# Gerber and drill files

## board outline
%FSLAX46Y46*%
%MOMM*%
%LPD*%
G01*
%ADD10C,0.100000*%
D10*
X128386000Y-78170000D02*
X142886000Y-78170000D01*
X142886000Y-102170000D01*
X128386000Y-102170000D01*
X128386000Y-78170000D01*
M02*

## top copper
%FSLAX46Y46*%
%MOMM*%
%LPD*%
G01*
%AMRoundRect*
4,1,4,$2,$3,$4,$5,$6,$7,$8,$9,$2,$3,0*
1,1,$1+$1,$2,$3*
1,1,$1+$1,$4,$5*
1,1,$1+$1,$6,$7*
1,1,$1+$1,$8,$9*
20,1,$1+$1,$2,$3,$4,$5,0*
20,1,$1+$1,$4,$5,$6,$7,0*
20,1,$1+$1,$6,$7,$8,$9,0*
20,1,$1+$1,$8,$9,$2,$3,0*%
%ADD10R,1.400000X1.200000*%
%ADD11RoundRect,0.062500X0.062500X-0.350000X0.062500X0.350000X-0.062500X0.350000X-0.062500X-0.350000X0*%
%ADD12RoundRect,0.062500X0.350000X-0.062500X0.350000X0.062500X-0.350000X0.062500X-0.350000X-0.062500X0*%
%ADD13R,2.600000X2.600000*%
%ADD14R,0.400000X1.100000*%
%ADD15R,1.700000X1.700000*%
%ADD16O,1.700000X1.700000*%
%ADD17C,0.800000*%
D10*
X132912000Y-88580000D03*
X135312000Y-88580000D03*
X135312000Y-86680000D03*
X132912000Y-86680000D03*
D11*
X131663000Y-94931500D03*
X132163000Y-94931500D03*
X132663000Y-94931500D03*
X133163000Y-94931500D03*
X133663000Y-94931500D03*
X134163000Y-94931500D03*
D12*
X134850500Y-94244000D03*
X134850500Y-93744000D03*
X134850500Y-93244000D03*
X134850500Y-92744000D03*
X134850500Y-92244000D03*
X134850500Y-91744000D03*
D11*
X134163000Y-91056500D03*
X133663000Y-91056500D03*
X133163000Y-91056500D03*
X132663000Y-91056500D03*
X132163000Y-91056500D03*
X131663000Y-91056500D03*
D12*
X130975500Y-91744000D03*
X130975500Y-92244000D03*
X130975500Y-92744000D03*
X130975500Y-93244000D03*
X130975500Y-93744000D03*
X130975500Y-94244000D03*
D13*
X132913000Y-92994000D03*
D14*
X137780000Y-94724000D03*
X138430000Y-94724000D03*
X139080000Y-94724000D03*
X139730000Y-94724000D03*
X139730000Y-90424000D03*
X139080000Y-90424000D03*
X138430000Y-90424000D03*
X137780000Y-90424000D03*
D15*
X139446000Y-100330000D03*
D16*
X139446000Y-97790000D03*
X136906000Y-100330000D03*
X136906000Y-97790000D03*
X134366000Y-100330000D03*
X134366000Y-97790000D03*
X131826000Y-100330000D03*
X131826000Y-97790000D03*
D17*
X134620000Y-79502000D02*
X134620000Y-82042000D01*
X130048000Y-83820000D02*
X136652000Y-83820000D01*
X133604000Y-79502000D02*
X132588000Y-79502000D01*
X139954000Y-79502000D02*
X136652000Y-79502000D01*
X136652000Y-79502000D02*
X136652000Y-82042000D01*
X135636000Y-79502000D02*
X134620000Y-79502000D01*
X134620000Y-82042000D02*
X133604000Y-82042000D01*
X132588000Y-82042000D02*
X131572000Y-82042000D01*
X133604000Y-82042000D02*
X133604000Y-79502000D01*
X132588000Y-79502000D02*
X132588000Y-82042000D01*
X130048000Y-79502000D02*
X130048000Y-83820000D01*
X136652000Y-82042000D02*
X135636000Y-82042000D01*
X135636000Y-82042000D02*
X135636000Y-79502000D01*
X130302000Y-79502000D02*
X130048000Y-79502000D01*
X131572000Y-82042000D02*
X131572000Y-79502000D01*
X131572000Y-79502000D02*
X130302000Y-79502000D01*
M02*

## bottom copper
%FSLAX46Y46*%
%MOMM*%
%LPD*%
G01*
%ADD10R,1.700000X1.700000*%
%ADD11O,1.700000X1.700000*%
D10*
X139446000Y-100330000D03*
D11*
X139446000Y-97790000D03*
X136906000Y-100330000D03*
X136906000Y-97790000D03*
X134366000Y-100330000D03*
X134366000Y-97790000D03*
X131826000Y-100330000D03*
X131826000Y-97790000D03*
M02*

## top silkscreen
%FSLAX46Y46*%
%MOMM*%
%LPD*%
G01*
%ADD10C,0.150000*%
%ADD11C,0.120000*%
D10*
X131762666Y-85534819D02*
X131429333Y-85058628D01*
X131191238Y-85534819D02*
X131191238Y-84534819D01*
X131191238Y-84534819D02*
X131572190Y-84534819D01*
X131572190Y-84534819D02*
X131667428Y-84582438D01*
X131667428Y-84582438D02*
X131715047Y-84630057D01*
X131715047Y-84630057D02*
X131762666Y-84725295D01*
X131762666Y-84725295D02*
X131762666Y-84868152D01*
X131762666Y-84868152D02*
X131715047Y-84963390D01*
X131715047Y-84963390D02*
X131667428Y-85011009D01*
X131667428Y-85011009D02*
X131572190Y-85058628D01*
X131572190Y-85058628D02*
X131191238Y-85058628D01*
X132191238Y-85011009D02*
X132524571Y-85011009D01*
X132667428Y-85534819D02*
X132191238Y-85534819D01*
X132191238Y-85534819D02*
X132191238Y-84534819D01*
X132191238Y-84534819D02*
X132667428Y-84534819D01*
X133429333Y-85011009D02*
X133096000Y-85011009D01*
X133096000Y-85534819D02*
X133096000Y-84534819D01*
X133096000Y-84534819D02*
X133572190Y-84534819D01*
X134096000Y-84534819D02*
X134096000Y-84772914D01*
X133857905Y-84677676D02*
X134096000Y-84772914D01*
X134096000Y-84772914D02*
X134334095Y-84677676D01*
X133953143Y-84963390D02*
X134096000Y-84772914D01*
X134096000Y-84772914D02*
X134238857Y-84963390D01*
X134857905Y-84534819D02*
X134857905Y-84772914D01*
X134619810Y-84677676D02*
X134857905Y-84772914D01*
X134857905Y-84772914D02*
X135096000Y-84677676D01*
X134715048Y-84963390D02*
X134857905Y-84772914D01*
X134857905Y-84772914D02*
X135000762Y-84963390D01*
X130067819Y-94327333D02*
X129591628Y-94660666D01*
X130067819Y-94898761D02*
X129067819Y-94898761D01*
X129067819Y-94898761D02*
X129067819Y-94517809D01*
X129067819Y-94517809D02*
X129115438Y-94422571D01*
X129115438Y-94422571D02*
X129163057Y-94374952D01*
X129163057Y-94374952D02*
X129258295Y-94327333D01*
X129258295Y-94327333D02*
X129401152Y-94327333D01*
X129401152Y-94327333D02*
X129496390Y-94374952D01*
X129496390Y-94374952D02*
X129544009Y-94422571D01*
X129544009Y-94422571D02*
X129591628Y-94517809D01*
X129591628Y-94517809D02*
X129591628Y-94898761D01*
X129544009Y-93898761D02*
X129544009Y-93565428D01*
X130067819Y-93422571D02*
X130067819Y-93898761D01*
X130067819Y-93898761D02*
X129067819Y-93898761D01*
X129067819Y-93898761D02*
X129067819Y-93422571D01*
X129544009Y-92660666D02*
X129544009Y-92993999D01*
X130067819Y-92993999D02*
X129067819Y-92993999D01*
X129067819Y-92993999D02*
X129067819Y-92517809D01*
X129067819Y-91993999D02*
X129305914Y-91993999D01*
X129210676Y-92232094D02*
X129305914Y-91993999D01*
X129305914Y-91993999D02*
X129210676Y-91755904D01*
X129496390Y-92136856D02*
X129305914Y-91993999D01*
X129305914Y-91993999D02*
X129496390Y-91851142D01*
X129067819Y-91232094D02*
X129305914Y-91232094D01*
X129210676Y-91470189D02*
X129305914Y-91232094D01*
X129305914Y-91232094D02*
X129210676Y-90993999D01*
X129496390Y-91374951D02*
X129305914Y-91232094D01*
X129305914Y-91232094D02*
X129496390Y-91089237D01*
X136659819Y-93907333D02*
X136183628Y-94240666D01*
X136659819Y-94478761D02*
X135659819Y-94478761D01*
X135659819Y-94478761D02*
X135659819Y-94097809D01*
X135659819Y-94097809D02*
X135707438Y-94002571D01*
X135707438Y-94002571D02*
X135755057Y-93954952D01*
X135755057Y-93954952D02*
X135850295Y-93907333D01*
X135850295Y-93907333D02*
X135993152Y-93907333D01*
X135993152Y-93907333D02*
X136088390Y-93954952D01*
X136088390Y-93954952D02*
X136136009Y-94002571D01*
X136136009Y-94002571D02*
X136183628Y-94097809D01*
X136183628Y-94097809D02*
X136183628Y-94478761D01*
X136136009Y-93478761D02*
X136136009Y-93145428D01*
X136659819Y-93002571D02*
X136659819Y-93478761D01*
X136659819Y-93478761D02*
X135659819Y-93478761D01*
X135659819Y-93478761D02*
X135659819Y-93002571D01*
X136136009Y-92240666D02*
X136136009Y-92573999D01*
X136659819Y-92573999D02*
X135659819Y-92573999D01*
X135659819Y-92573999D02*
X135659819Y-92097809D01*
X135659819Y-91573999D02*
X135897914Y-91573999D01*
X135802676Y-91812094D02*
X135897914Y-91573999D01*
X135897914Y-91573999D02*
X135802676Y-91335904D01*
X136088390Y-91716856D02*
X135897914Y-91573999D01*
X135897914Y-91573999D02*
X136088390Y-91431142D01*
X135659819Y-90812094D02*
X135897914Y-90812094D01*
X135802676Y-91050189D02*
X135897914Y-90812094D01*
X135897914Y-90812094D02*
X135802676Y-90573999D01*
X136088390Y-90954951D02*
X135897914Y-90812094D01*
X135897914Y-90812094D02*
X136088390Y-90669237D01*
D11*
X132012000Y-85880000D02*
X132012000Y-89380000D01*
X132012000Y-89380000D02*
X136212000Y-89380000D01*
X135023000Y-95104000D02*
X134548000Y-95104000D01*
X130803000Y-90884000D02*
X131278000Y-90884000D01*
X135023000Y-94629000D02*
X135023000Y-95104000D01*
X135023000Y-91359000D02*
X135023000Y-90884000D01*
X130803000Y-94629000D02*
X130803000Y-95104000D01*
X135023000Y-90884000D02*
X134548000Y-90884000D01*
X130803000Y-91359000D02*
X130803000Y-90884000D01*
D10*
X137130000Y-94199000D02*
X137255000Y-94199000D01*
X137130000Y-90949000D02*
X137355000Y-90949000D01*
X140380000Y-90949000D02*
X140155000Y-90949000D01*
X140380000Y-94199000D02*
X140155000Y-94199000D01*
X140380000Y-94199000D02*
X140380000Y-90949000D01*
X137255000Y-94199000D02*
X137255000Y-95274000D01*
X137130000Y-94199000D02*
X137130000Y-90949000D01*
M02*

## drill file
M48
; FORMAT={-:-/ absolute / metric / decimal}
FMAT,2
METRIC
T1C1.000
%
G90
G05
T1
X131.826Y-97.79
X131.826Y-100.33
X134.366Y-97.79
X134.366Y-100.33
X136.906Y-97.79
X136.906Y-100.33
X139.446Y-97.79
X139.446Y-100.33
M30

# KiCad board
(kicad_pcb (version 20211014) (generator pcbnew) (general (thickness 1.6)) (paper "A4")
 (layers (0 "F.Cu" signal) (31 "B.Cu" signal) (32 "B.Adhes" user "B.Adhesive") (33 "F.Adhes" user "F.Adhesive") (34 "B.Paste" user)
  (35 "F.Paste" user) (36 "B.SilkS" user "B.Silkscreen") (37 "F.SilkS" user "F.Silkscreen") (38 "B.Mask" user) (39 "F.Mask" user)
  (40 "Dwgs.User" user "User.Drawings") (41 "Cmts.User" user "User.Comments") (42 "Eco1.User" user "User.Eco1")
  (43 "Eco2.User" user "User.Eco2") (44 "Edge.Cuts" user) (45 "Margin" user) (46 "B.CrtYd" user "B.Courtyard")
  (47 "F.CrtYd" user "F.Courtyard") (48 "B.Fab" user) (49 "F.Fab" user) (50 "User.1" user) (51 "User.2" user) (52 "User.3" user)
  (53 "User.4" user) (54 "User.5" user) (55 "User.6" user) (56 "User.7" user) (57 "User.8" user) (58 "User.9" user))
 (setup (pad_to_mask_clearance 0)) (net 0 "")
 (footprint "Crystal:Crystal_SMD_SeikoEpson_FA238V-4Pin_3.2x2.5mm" (layer "F.Cu") (at 134.112 87.63)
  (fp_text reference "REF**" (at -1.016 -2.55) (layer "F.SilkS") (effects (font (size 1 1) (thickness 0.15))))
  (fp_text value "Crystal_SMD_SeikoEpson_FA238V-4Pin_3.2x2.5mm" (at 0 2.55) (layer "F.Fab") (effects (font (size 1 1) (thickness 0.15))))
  (fp_line (start -2.1 -1.75) (end -2.1 1.75) (layer "F.SilkS") (width 0.12))
  (fp_line (start -2.1 1.75) (end 2.1 1.75) (layer "F.SilkS") (width 0.12))
  (pad "1" smd rect (at -1.2 0.95) (size 1.4 1.2) (layers "F.Cu" "F.Paste" "F.Mask"))
  (pad "2" smd rect (at 1.2 0.95) (size 1.4 1.2) (layers "F.Cu" "F.Paste" "F.Mask"))
  (pad "3" smd rect (at 1.2 -0.95) (size 1.4 1.2) (layers "F.Cu" "F.Paste" "F.Mask"))
  (pad "4" smd rect (at -1.2 -0.95) (size 1.4 1.2) (layers "F.Cu" "F.Paste" "F.Mask")))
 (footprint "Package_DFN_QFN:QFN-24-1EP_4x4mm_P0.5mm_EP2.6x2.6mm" (layer "F.Cu") (at 132.913 92.994 90)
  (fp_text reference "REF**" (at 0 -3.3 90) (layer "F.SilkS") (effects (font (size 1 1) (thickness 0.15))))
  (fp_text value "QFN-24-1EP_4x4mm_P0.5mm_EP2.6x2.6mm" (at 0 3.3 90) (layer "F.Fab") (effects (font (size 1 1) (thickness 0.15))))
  (fp_line (start -2.11 2.11) (end -2.11 1.635) (layer "F.SilkS") (width 0.12))
  (fp_line (start 2.11 -2.11) (end 2.11 -1.635) (layer "F.SilkS") (width 0.12))
  (fp_line (start -1.635 2.11) (end -2.11 2.11) (layer "F.SilkS") (width 0.12))
  (fp_line (start 1.635 2.11) (end 2.11 2.11) (layer "F.SilkS") (width 0.12))
  (fp_line (start -1.635 -2.11) (end -2.11 -2.11) (layer "F.SilkS") (width 0.12))
  (fp_line (start 2.11 2.11) (end 2.11 1.635) (layer "F.SilkS") (width 0.12))
  (fp_line (start 1.635 -2.11) (end 2.11 -2.11) (layer "F.SilkS") (width 0.12))
  (pad "" smd roundrect (at -0.65 -0.65 90) (size 1.05 1.05) (layers "F.Paste") (roundrect_rratio 0.238095))
  (pad "" smd roundrect (at 0.65 0.65 90) (size 1.05 1.05) (layers "F.Paste") (roundrect_rratio 0.238095))
  (pad "" smd roundrect (at 0.65 -0.65 90) (size 1.05 1.05) (layers "F.Paste") (roundrect_rratio 0.238095))
  (pad "" smd roundrect (at -0.65 0.65 90) (size 1.05 1.05) (layers "F.Paste") (roundrect_rratio 0.238095))
  (pad "1" smd roundrect (at -1.9375 -1.25 90) (size 0.825 0.25) (layers "F.Cu" "F.Paste" "F.Mask") (roundrect_rratio 0.25))
  (pad "2" smd roundrect (at -1.9375 -0.75 90) (size 0.825 0.25) (layers "F.Cu" "F.Paste" "F.Mask") (roundrect_rratio 0.25))
  (pad "3" smd roundrect (at -1.9375 -0.25 90) (size 0.825 0.25) (layers "F.Cu" "F.Paste" "F.Mask") (roundrect_rratio 0.25))
  (pad "4" smd roundrect (at -1.9375 0.25 90) (size 0.825 0.25) (layers "F.Cu" "F.Paste" "F.Mask") (roundrect_rratio 0.25))
  (pad "5" smd roundrect (at -1.9375 0.75 90) (size 0.825 0.25) (layers "F.Cu" "F.Paste" "F.Mask") (roundrect_rratio 0.25))
  (pad "6" smd roundrect (at -1.9375 1.25 90) (size 0.825 0.25) (layers "F.Cu" "F.Paste" "F.Mask") (roundrect_rratio 0.25))
  (pad "7" smd roundrect (at -1.25 1.9375 90) (size 0.25 0.825) (layers "F.Cu" "F.Paste" "F.Mask") (roundrect_rratio 0.25))
  (pad "8" smd roundrect (at -0.75 1.9375 90) (size 0.25 0.825) (layers "F.Cu" "F.Paste" "F.Mask") (roundrect_rratio 0.25))
  (pad "9" smd roundrect (at -0.25 1.9375 90) (size 0.25 0.825) (layers "F.Cu" "F.Paste" "F.Mask") (roundrect_rratio 0.25))
  (pad "10" smd roundrect (at 0.25 1.9375 90) (size 0.25 0.825) (layers "F.Cu" "F.Paste" "F.Mask") (roundrect_rratio 0.25))
  (pad "11" smd roundrect (at 0.75 1.9375 90) (size 0.25 0.825) (layers "F.Cu" "F.Paste" "F.Mask") (roundrect_rratio 0.25))
  (pad "12" smd roundrect (at 1.25 1.9375 90) (size 0.25 0.825) (layers "F.Cu" "F.Paste" "F.Mask") (roundrect_rratio 0.25))
  (pad "13" smd roundrect (at 1.9375 1.25 90) (size 0.825 0.25) (layers "F.Cu" "F.Paste" "F.Mask") (roundrect_rratio 0.25))
  (pad "14" smd roundrect (at 1.9375 0.75 90) (size 0.825 0.25) (layers "F.Cu" "F.Paste" "F.Mask") (roundrect_rratio 0.25))
  (pad "15" smd roundrect (at 1.9375 0.25 90) (size 0.825 0.25) (layers "F.Cu" "F.Paste" "F.Mask") (roundrect_rratio 0.25))
  (pad "16" smd roundrect (at 1.9375 -0.25 90) (size 0.825 0.25) (layers "F.Cu" "F.Paste" "F.Mask") (roundrect_rratio 0.25))
  (pad "17" smd roundrect (at 1.9375 -0.75 90) (size 0.825 0.25) (layers "F.Cu" "F.Paste" "F.Mask") (roundrect_rratio 0.25))
  (pad "18" smd roundrect (at 1.9375 -1.25 90) (size 0.825 0.25) (layers "F.Cu" "F.Paste" "F.Mask") (roundrect_rratio 0.25))
  (pad "19" smd roundrect (at 1.25 -1.9375 90) (size 0.25 0.825) (layers "F.Cu" "F.Paste" "F.Mask") (roundrect_rratio 0.25))
  (pad "20" smd roundrect (at 0.75 -1.9375 90) (size 0.25 0.825) (layers "F.Cu" "F.Paste" "F.Mask") (roundrect_rratio 0.25))
  (pad "21" smd roundrect (at 0.25 -1.9375 90) (size 0.25 0.825) (layers "F.Cu" "F.Paste" "F.Mask") (roundrect_rratio 0.25))
  (pad "22" smd roundrect (at -0.25 -1.9375 90) (size 0.25 0.825) (layers "F.Cu" "F.Paste" "F.Mask") (roundrect_rratio 0.25))
  (pad "23" smd roundrect (at -0.75 -1.9375 90) (size 0.25 0.825) (layers "F.Cu" "F.Paste" "F.Mask") (roundrect_rratio 0.25))
  (pad "24" smd roundrect (at -1.25 -1.9375 90) (size 0.25 0.825) (layers "F.Cu" "F.Paste" "F.Mask") (roundrect_rratio 0.25))
  (pad "25" smd rect (at 0 0 90) (size 2.6 2.6) (layers "F.Cu" "F.Mask")))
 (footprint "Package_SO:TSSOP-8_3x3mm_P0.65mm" (layer "F.Cu") (at 138.755 92.574 90)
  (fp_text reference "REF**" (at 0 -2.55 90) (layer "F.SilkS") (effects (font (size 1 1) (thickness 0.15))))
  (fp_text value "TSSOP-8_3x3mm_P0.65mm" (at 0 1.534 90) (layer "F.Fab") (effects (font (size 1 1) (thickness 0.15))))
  (fp_line (start -1.625 -1.625) (end -1.625 -1.5) (layer "F.SilkS") (width 0.15))
  (fp_line (start 1.625 -1.625) (end 1.625 -1.4) (layer "F.SilkS") (width 0.15))
  (fp_line (start 1.625 1.625) (end 1.625 1.4) (layer "F.SilkS") (width 0.15))
  (fp_line (start -1.625 1.625) (end -1.625 1.4) (layer "F.SilkS") (width 0.15))
  (fp_line (start -1.625 1.625) (end 1.625 1.625) (layer "F.SilkS") (width 0.15))
  (fp_line (start -1.625 -1.5) (end -2.7 -1.5) (layer "F.SilkS") (width 0.15))
  (fp_line (start -1.625 -1.625) (end 1.625 -1.625) (layer "F.SilkS") (width 0.15))
  (pad "1" smd rect (at -2.15 -0.975 90) (size 1.1 0.4) (layers "F.Cu" "F.Paste" "F.Mask"))
  (pad "2" smd rect (at -2.15 -0.325 90) (size 1.1 0.4) (layers "F.Cu" "F.Paste" "F.Mask"))
  (pad "3" smd rect (at -2.15 0.325 90) (size 1.1 0.4) (layers "F.Cu" "F.Paste" "F.Mask"))
  (pad "4" smd rect (at -2.15 0.975 90) (size 1.1 0.4) (layers "F.Cu" "F.Paste" "F.Mask"))
  (pad "5" smd rect (at 2.15 0.975 90) (size 1.1 0.4) (layers "F.Cu" "F.Paste" "F.Mask"))
  (pad "6" smd rect (at 2.15 0.325 90) (size 1.1 0.4) (layers "F.Cu" "F.Paste" "F.Mask"))
  (pad "7" smd rect (at 2.15 -0.325 90) (size 1.1 0.4) (layers "F.Cu" "F.Paste" "F.Mask"))
  (pad "8" smd rect (at 2.15 -0.975 90) (size 1.1 0.4) (layers "F.Cu" "F.Paste" "F.Mask")))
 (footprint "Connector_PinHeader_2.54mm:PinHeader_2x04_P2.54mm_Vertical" (layer "B.Cu") (at 139.446 100.33 90)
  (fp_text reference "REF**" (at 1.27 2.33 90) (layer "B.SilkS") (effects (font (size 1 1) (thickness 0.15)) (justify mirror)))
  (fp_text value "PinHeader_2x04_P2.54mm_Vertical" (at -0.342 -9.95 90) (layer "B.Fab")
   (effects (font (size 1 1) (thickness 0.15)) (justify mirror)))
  (pad "1" thru_hole rect (at 0 0 90) (size 1.7 1.7) (drill 1) (layers *.Cu *.Mask))
  (pad "2" thru_hole oval (at 2.54 0 90) (size 1.7 1.7) (drill 1) (layers *.Cu *.Mask))
  (pad "3" thru_hole oval (at 0 -2.54 90) (size 1.7 1.7) (drill 1) (layers *.Cu *.Mask))
  (pad "4" thru_hole oval (at 2.54 -2.54 90) (size 1.7 1.7) (drill 1) (layers *.Cu *.Mask))
  (pad "5" thru_hole oval (at 0 -5.08 90) (size 1.7 1.7) (drill 1) (layers *.Cu *.Mask))
  (pad "6" thru_hole oval (at 2.54 -5.08 90) (size 1.7 1.7) (drill 1) (layers *.Cu *.Mask))
  (pad "7" thru_hole oval (at 0 -7.62 90) (size 1.7 1.7) (drill 1) (layers *.Cu *.Mask))
  (pad "8" thru_hole oval (at 2.54 -7.62 90) (size 1.7 1.7) (drill 1) (layers *.Cu *.Mask)))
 (gr_rect (start 128.386 78.17) (end 142.886 102.17) (layer "Edge.Cuts") (width 0.1) (fill none))
 (segment (start 134.62 79.502) (end 134.62 82.042) (width 0.8) (layer "F.Cu") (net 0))
 (segment (start 130.048 83.82) (end 136.652 83.82) (width 0.8) (layer "F.Cu") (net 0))
 (segment (start 133.604 79.502) (end 132.588 79.502) (width 0.8) (layer "F.Cu") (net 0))
 (segment (start 139.954 79.502) (end 136.652 79.502) (width 0.8) (layer "F.Cu") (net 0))
 (segment (start 136.652 79.502) (end 136.652 82.042) (width 0.8) (layer "F.Cu") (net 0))
 (segment (start 135.636 79.502) (end 134.62 79.502) (width 0.8) (layer "F.Cu") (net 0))
 (segment (start 134.62 82.042) (end 133.604 82.042) (width 0.8) (layer "F.Cu") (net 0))
 (segment (start 132.588 82.042) (end 131.572 82.042) (width 0.8) (layer "F.Cu") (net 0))
 (segment (start 133.604 82.042) (end 133.604 79.502) (width 0.8) (layer "F.Cu") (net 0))
 (segment (start 132.588 79.502) (end 132.588 82.042) (width 0.8) (layer "F.Cu") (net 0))
 (segment (start 130.048 79.502) (end 130.048 83.82) (width 0.8) (layer "F.Cu") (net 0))
 (segment (start 136.652 82.042) (end 135.636 82.042) (width 0.8) (layer "F.Cu") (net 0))
 (segment (start 135.636 82.042) (end 135.636 79.502) (width 0.8) (layer "F.Cu") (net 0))
 (segment (start 130.302 79.502) (end 130.048 79.502) (width 0.8) (layer "F.Cu") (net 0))
 (segment (start 131.572 82.042) (end 131.572 79.502) (width 0.8) (layer "F.Cu") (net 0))
 (segment (start 131.572 79.502) (end 130.302 79.502) (width 0.8) (layer "F.Cu") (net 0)))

